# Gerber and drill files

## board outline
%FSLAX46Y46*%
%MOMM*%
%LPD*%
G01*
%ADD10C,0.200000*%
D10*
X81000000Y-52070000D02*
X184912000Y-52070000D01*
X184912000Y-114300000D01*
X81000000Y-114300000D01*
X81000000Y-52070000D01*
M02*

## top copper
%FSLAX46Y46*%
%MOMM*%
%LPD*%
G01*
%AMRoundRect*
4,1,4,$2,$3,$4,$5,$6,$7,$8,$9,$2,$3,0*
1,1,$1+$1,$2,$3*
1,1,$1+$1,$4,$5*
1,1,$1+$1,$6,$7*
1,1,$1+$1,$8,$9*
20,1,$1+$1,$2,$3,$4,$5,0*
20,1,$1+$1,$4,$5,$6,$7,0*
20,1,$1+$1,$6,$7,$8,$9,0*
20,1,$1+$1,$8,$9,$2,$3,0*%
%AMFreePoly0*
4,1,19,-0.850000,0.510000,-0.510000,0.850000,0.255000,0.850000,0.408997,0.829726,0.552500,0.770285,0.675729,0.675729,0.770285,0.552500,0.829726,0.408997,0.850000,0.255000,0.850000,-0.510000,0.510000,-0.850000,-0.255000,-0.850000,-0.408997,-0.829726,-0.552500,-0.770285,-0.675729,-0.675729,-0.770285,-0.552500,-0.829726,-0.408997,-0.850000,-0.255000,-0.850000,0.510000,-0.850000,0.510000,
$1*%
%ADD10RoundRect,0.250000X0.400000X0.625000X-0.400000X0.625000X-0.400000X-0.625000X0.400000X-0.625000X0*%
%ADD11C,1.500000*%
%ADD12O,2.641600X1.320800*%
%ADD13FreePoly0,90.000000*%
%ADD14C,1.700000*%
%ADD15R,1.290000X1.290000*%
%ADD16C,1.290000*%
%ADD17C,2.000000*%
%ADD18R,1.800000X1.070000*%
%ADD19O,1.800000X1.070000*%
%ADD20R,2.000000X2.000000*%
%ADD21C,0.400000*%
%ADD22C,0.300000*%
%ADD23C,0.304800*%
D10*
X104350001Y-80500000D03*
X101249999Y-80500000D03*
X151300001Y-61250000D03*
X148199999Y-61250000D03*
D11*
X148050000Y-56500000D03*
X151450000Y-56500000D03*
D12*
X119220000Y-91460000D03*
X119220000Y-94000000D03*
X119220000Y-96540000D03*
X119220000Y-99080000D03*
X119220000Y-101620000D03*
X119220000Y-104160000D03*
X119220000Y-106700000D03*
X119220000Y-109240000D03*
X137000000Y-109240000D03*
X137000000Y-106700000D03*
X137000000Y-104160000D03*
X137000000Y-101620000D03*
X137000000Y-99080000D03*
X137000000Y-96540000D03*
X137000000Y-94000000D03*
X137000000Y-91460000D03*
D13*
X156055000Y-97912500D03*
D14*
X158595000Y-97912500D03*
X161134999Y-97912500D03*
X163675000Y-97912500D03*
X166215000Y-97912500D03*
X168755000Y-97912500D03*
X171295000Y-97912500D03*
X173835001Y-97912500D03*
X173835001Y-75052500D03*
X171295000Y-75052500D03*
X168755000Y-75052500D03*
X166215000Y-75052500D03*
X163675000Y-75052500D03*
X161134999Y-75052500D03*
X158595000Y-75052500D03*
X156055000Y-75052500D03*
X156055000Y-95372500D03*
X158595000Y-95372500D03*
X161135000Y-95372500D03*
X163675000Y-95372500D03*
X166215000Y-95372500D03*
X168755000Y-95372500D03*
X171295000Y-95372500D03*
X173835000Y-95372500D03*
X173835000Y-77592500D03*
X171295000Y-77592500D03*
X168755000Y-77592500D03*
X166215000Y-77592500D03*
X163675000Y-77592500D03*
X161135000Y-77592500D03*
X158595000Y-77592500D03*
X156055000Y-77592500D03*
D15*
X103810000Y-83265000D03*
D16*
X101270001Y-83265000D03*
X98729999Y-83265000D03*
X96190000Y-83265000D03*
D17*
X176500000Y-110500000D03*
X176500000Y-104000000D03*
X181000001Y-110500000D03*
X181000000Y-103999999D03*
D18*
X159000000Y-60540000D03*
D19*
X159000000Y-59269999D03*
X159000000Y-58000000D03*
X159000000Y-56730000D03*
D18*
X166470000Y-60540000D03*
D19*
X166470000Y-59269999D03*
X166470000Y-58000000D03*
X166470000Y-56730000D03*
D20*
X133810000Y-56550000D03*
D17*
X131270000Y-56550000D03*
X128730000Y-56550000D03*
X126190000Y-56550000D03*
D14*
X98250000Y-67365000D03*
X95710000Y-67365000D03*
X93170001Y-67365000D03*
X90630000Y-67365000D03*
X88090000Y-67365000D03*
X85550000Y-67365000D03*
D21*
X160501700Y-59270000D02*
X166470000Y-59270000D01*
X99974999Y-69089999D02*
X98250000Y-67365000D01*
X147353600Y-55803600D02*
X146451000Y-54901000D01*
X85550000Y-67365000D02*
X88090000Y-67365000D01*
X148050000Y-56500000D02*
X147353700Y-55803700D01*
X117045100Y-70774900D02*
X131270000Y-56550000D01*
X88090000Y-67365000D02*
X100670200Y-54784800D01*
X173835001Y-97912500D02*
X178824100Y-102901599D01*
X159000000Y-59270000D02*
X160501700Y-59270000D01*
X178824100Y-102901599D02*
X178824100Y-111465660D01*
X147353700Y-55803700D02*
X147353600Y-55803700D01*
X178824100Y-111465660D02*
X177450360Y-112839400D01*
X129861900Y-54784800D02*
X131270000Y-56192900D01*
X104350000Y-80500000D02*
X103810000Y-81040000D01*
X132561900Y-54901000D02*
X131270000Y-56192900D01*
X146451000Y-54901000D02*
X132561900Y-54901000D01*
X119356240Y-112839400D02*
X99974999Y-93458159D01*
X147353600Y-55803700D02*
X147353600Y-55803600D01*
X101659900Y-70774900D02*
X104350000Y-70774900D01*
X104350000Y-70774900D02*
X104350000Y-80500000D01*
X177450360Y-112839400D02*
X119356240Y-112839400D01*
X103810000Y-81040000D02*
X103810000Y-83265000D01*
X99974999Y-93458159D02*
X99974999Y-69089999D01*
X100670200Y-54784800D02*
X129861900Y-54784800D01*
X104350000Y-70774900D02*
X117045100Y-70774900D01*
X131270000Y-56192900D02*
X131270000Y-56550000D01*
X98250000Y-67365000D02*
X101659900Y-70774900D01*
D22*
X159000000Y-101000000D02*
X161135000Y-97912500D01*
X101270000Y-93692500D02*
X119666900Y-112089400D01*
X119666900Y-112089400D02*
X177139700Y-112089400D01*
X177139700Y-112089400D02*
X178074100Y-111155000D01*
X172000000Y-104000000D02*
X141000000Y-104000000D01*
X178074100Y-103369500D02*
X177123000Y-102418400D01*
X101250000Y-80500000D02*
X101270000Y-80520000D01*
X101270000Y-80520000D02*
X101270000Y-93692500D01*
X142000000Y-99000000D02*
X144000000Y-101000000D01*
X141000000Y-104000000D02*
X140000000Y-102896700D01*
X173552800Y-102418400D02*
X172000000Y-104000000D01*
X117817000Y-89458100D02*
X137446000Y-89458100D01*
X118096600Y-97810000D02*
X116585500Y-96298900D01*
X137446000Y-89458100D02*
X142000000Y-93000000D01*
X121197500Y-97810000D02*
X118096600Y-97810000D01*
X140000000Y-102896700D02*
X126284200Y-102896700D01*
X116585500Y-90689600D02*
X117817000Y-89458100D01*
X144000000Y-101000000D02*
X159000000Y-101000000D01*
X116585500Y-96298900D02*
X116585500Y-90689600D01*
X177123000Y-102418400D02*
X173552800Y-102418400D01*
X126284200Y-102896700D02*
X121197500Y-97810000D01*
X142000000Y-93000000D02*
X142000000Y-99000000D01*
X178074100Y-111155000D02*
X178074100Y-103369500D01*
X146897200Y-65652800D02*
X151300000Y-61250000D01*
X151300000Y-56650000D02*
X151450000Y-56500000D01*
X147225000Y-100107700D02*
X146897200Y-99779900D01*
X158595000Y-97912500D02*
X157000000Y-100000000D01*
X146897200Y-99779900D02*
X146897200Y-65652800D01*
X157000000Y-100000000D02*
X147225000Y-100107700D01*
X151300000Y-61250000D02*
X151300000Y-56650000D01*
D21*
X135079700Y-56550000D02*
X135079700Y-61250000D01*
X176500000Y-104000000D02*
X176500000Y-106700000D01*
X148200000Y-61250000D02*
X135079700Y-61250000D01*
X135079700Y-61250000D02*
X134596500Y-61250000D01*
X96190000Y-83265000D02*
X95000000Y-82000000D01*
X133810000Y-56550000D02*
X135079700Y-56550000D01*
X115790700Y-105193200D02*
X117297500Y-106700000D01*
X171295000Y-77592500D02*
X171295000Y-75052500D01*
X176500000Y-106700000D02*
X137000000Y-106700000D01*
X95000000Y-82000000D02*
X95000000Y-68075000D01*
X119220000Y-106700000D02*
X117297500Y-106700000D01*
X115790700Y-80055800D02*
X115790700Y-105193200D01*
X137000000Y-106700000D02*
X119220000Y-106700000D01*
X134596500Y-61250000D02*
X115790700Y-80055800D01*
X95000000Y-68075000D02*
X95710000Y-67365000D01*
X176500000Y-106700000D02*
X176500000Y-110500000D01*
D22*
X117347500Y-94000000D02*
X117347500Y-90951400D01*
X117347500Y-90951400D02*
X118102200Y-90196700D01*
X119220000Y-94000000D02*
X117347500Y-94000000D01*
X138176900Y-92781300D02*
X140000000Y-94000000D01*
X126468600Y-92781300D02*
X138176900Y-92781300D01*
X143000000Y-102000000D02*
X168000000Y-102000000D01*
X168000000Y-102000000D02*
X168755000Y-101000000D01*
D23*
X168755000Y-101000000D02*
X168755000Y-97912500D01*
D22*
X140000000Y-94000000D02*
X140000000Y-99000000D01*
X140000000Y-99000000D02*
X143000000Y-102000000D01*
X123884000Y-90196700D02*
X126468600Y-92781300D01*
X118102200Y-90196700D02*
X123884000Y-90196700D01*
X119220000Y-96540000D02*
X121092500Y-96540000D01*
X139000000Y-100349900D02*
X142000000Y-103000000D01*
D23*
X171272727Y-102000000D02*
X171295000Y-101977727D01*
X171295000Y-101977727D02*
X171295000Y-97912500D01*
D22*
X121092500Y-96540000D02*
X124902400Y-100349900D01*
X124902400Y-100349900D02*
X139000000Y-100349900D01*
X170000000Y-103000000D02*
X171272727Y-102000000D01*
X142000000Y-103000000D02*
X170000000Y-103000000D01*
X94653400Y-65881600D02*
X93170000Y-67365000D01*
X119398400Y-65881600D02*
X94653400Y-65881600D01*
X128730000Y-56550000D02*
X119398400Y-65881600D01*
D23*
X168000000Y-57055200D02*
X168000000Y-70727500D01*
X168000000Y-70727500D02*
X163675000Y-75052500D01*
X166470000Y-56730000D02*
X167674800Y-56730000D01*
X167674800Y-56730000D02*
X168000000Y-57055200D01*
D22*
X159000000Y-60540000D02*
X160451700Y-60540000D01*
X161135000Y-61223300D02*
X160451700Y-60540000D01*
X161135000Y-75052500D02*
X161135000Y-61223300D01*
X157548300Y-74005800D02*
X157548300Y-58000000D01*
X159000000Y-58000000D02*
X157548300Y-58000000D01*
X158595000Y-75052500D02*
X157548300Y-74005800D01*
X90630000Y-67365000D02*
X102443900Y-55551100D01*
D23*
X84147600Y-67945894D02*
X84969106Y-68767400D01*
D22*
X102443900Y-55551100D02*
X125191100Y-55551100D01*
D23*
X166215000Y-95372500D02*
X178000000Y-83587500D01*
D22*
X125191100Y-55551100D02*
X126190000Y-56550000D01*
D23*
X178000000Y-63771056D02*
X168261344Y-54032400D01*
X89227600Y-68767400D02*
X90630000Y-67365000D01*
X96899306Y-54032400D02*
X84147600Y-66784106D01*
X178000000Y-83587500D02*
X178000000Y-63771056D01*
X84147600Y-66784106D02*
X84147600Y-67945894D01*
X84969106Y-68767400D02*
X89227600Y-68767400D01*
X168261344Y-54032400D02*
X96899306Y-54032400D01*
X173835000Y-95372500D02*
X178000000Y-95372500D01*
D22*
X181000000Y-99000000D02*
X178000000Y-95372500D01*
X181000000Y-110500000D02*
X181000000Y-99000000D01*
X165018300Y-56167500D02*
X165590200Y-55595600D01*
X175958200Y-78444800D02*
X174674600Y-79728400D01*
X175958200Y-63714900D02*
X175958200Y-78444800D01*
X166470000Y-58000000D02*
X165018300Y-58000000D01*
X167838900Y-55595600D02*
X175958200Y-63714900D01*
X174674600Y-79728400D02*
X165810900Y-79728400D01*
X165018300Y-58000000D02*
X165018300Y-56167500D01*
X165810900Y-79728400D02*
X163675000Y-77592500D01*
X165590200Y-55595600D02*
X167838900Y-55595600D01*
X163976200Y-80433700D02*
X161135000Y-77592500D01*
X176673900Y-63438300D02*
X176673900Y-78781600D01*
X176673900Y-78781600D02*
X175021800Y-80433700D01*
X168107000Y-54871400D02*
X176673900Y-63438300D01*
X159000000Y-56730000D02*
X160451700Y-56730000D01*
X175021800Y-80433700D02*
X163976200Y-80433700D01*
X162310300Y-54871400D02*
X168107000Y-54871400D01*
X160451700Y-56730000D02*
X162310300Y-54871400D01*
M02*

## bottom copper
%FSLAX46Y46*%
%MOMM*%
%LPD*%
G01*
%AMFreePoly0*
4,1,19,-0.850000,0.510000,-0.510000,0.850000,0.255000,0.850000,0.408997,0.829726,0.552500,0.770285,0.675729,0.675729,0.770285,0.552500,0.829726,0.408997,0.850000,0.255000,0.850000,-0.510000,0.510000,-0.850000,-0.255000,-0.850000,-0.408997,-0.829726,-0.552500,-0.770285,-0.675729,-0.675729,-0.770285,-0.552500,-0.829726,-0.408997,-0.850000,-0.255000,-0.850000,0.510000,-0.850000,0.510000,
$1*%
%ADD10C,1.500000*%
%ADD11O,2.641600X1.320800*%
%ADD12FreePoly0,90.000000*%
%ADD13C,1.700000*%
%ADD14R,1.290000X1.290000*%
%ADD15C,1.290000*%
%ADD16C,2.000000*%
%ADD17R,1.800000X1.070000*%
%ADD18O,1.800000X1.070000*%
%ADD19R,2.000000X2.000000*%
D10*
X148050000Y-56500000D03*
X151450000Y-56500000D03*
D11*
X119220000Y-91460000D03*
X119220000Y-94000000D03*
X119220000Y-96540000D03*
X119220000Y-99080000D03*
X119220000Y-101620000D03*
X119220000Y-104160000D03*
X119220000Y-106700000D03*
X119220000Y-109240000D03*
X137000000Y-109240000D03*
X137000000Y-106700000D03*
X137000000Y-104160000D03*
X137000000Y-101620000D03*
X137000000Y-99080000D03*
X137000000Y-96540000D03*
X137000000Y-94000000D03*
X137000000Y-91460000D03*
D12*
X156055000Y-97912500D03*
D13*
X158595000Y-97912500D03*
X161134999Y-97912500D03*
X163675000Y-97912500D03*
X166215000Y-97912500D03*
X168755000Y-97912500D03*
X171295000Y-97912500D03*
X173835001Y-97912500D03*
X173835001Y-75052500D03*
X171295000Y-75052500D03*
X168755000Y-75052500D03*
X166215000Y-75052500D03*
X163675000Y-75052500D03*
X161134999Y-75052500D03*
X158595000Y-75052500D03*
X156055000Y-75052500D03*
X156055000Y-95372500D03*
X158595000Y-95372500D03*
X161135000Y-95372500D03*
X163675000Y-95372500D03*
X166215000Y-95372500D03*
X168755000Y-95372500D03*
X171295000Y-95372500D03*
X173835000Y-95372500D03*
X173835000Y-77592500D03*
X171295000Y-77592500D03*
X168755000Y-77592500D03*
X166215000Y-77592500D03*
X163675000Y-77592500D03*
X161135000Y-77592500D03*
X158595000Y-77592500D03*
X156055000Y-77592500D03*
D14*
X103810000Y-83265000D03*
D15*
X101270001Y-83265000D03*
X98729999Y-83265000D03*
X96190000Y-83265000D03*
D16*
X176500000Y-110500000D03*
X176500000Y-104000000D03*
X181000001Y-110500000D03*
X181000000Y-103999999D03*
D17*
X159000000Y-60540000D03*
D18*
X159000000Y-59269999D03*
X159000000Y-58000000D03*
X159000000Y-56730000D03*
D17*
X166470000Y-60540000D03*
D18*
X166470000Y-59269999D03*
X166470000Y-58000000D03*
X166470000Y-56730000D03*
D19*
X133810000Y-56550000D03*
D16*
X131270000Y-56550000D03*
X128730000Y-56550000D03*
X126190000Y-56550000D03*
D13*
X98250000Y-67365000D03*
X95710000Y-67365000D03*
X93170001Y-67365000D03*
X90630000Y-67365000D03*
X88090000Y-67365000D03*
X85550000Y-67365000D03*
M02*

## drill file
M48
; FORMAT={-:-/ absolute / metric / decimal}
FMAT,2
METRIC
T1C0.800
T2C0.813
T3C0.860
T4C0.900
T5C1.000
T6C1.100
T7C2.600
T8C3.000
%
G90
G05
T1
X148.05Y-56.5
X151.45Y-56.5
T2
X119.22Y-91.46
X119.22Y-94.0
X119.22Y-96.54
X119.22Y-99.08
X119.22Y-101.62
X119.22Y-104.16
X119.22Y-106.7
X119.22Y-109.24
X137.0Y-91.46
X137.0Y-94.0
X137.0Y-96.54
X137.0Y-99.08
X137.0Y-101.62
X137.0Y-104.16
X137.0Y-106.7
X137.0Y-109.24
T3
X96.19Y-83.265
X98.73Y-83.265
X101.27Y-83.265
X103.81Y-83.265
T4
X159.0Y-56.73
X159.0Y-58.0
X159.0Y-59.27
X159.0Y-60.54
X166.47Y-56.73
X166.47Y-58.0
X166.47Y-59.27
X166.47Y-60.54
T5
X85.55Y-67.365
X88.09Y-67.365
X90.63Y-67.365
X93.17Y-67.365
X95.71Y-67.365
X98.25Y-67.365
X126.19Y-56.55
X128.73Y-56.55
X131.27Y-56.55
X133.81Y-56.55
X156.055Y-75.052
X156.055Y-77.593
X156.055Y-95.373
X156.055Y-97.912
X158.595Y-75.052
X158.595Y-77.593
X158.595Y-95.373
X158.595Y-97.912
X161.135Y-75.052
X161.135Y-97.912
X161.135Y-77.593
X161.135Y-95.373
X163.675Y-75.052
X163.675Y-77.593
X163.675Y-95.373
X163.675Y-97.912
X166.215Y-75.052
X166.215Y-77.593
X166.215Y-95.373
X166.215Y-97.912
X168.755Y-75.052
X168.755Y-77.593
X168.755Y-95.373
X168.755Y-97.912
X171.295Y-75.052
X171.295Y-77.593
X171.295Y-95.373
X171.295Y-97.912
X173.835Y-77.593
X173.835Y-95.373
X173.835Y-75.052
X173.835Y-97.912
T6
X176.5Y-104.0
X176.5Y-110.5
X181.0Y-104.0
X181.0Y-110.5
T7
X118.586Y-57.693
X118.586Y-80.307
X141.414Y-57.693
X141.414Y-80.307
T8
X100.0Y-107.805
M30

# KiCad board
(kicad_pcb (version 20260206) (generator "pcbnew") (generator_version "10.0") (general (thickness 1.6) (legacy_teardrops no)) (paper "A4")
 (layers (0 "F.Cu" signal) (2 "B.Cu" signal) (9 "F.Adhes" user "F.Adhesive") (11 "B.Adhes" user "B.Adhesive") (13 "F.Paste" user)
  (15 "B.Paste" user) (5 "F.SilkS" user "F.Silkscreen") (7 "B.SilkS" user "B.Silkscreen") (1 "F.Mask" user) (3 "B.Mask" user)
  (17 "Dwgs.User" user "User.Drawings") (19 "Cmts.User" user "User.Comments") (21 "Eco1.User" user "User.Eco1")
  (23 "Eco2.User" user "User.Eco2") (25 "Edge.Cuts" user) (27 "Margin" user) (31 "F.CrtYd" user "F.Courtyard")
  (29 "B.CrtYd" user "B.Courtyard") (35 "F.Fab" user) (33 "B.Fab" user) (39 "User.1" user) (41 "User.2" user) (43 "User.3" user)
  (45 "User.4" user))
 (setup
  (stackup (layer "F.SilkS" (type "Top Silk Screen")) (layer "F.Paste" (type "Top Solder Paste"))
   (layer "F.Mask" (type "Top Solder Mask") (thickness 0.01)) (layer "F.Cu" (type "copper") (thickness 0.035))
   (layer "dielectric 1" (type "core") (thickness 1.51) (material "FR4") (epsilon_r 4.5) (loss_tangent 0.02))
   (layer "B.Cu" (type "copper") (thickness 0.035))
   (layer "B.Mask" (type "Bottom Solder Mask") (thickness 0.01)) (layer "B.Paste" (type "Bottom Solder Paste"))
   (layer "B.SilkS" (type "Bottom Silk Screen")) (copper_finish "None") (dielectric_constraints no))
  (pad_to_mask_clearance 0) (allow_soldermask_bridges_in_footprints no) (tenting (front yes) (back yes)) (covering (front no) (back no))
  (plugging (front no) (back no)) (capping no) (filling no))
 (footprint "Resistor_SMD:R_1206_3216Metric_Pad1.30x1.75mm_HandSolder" (layer "F.Cu") (at 102.8 80.5 180)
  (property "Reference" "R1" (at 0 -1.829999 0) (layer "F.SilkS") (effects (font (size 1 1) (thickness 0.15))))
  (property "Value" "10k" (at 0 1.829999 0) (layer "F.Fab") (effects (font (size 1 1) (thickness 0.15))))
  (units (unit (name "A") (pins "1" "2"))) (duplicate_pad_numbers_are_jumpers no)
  (pad "1" smd roundrect (at -1.550001 0 180) (size 1.3 1.75) (layers "F.Cu" "F.Mask" "F.Paste") (roundrect_rratio 0.192308) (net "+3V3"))
  (pad "2" smd roundrect (at 1.550001 0 180) (size 1.3 1.75) (layers "F.Cu" "F.Mask" "F.Paste") (roundrect_rratio 0.192308)
   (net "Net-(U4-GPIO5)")))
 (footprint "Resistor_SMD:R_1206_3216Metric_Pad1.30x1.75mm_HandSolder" (layer "F.Cu") (at 149.75 61.25 180)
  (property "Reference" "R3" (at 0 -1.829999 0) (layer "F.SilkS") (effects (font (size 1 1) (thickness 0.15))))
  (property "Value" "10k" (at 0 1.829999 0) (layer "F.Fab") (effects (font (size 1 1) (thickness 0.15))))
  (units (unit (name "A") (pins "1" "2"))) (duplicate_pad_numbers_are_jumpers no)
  (pad "1" smd roundrect (at -1.550001 0 180) (size 1.3 1.75) (layers "F.Cu" "F.Mask" "F.Paste") (roundrect_rratio 0.192308)
   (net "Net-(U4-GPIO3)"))
  (pad "2" smd roundrect (at 1.550001 0 180) (size 1.3 1.75) (layers "F.Cu" "F.Mask" "F.Paste") (roundrect_rratio 0.192308) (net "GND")))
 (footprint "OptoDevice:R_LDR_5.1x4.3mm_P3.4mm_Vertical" (layer "F.Cu") (at 148.05 56.5)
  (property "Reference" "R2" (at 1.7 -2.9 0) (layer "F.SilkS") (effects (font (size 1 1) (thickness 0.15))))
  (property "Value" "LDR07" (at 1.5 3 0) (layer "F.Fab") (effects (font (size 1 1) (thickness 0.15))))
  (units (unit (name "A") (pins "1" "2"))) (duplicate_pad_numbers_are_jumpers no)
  (pad "1" thru_hole circle (at 0 0) (size 1.5 1.5) (drill 0.8) (layers "*.Cu" "*.Mask") (remove_unused_layers no) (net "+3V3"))
  (pad "2" thru_hole circle (at 3.4 0) (size 1.5 1.5) (drill 0.8) (layers "*.Cu" "*.Mask") (remove_unused_layers no) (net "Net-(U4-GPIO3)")))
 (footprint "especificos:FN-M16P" (layer "F.Cu") (at 128.11 100.35 -90)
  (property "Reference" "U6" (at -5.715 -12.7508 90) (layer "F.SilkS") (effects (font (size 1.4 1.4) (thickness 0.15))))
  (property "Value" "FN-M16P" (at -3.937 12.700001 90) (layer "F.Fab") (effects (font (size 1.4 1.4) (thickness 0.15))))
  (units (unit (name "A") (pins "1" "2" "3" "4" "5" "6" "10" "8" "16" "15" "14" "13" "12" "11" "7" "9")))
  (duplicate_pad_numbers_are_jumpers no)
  (pad "1" thru_hole oval (at -8.89 8.89 270) (size 1.3208 2.6416) (drill 0.8128) (layers "*.Cu" "*.Mask") (remove_unused_layers no)
   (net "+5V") (solder_mask_margin 0.102))
  (pad "2" thru_hole oval (at -6.35 8.89 270) (size 1.3208 2.6416) (drill 0.8128) (layers "*.Cu" "*.Mask") (remove_unused_layers no)
   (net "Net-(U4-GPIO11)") (solder_mask_margin 0.102))
  (pad "3" thru_hole oval (at -3.81 8.89 270) (size 1.3208 2.6416) (drill 0.8128) (layers "*.Cu" "*.Mask") (remove_unused_layers no)
   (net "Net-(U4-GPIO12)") (solder_mask_margin 0.102))
  (pad "4" thru_hole oval (at -1.27 8.89 270) (size 1.3208 2.6416) (drill 0.8128) (layers "*.Cu" "*.Mask") (remove_unused_layers no)
   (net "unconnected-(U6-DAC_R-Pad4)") (solder_mask_margin 0.102))
  (pad "5" thru_hole oval (at 1.27 8.89 270) (size 1.3208 2.6416) (drill 0.8128) (layers "*.Cu" "*.Mask") (remove_unused_layers no)
   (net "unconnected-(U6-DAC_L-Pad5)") (solder_mask_margin 0.102))
  (pad "6" thru_hole oval (at 3.81 8.89 270) (size 1.3208 2.6416) (drill 0.8128) (layers "*.Cu" "*.Mask") (remove_unused_layers no)
   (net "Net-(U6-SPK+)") (solder_mask_margin 0.102))
  (pad "7" thru_hole oval (at 6.35 8.89 270) (size 1.3208 2.6416) (drill 0.8128) (layers "*.Cu" "*.Mask") (remove_unused_layers no)
   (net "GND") (solder_mask_margin 0.102))
  (pad "8" thru_hole oval (at 8.89 8.89 270) (size 1.3208 2.6416) (drill 0.8128) (layers "*.Cu" "*.Mask") (remove_unused_layers no)
   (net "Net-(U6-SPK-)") (solder_mask_margin 0.102))
  (pad "9" thru_hole oval (at 8.89 -8.89 270) (size 1.3208 2.6416) (drill 0.8128) (layers "*.Cu" "*.Mask") (remove_unused_layers no)
   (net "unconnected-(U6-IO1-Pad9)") (solder_mask_margin 0.102))
  (pad "10" thru_hole oval (at 6.35 -8.89 270) (size 1.3208 2.6416) (drill 0.8128) (layers "*.Cu" "*.Mask") (remove_unused_layers no)
   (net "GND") (solder_mask_margin 0.102))
  (pad "11" thru_hole oval (at 3.81 -8.89 270) (size 1.3208 2.6416) (drill 0.8128) (layers "*.Cu" "*.Mask") (remove_unused_layers no)
   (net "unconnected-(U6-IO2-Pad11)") (solder_mask_margin 0.102))
  (pad "12" thru_hole oval (at 1.27 -8.89 270) (size 1.3208 2.6416) (drill 0.8128) (layers "*.Cu" "*.Mask") (remove_unused_layers no)
   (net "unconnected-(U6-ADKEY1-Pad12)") (solder_mask_margin 0.102))
  (pad "13" thru_hole oval (at -1.27 -8.89 270) (size 1.3208 2.6416) (drill 0.8128) (layers "*.Cu" "*.Mask") (remove_unused_layers no)
   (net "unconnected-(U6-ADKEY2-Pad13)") (solder_mask_margin 0.102))
  (pad "14" thru_hole oval (at -3.81 -8.89 270) (size 1.3208 2.6416) (drill 0.8128) (layers "*.Cu" "*.Mask") (remove_unused_layers no)
   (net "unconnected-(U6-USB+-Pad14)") (solder_mask_margin 0.102))
  (pad "15" thru_hole oval (at -6.35 -8.89 270) (size 1.3208 2.6416) (drill 0.8128) (layers "*.Cu" "*.Mask") (remove_unused_layers no)
   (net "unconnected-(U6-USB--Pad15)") (solder_mask_margin 0.102))
  (pad "16" thru_hole oval (at -8.89 -8.89 270) (size 1.3208 2.6416) (drill 0.8128) (layers "*.Cu" "*.Mask") (remove_unused_layers no)
   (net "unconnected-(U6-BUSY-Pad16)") (solder_mask_margin 0.102)))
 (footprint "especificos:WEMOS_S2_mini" (layer "F.Cu") (at 156.055 97.9125 90)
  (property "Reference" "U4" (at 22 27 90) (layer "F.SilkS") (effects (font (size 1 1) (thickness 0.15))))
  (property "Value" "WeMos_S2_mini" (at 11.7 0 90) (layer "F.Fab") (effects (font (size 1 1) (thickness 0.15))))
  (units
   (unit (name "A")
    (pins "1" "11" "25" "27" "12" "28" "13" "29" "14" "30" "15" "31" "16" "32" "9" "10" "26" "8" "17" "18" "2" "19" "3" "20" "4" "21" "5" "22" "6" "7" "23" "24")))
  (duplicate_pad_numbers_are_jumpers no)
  (pad "1" thru_hole roundrect (at 0 0 90) (size 1.7 1.7) (drill 1) (layers "*.Cu" "*.Mask") (remove_unused_layers no)
   (roundrect_rratio 0.35) (chamfer_ratio 0.2) (chamfer top_left bottom_right) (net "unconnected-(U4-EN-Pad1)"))
  (pad "2" thru_hole circle (at 0 2.54 90) (size 1.7 1.7) (drill 1) (layers "*.Cu" "*.Mask") (remove_unused_layers no)
   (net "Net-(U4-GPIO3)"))
  (pad "3" thru_hole circle (at 0 5.079999 90) (size 1.7 1.7) (drill 1) (layers "*.Cu" "*.Mask") (remove_unused_layers no)
   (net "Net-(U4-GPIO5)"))
  (pad "4" thru_hole circle (at 0 7.62 90) (size 1.7 1.7) (drill 1) (layers "*.Cu" "*.Mask") (remove_unused_layers no)
   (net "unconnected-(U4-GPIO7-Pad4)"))
  (pad "5" thru_hole circle (at 0 10.16 90) (size 1.7 1.7) (drill 1) (layers "*.Cu" "*.Mask") (remove_unused_layers no) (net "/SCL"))
  (pad "6" thru_hole circle (at 0 12.7 90) (size 1.7 1.7) (drill 1) (layers "*.Cu" "*.Mask") (remove_unused_layers no)
   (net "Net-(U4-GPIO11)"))
  (pad "7" thru_hole circle (at 0 15.24 90) (size 1.7 1.7) (drill 1) (layers "*.Cu" "*.Mask") (remove_unused_layers no)
   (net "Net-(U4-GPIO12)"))
  (pad "8" thru_hole circle (at 0 17.780001 90) (size 1.7 1.7) (drill 1) (layers "*.Cu" "*.Mask") (remove_unused_layers no) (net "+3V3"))
  (pad "9" thru_hole circle (at 22.86 17.780001 90) (size 1.7 1.7) (drill 1) (layers "*.Cu" "*.Mask") (remove_unused_layers no) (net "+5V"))
  (pad "10" thru_hole circle (at 22.86 15.24 90) (size 1.7 1.7) (drill 1) (layers "*.Cu" "*.Mask") (remove_unused_layers no) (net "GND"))
  (pad "11" thru_hole circle (at 22.86 12.7 90) (size 1.7 1.7) (drill 1) (layers "*.Cu" "*.Mask") (remove_unused_layers no)
   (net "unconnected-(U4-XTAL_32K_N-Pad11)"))
  (pad "12" thru_hole circle (at 22.86 10.16 90) (size 1.7 1.7) (drill 1) (layers "*.Cu" "*.Mask") (remove_unused_layers no)
   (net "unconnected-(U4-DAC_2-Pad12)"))
  (pad "13" thru_hole circle (at 22.86 7.62 90) (size 1.7 1.7) (drill 1) (layers "*.Cu" "*.Mask") (remove_unused_layers no)
   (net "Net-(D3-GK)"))
  (pad "14" thru_hole circle (at 22.86 5.079999 90) (size 1.7 1.7) (drill 1) (layers "*.Cu" "*.Mask") (remove_unused_layers no)
   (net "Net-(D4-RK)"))
  (pad "15" thru_hole circle (at 22.86 2.54 90) (size 1.7 1.7) (drill 1) (layers "*.Cu" "*.Mask") (remove_unused_layers no)
   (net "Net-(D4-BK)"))
  (pad "16" thru_hole circle (at 22.86 0 90) (size 1.7 1.7) (drill 1) (layers "*.Cu" "*.Mask") (remove_unused_layers no)
   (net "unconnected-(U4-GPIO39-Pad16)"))
  (pad "17" thru_hole circle (at 2.54 0 90) (size 1.7 1.7) (drill 1) (layers "*.Cu" "*.Mask") (remove_unused_layers no)
   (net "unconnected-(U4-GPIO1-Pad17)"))
  (pad "18" thru_hole circle (at 2.54 2.54 90) (size 1.7 1.7) (drill 1) (layers "*.Cu" "*.Mask") (remove_unused_layers no)
   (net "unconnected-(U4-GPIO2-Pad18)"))
  (pad "19" thru_hole circle (at 2.54 5.08 90) (size 1.7 1.7) (drill 1) (layers "*.Cu" "*.Mask") (remove_unused_layers no)
   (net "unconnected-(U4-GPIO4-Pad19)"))
  (pad "20" thru_hole circle (at 2.54 7.62 90) (size 1.7 1.7) (drill 1) (layers "*.Cu" "*.Mask") (remove_unused_layers no)
   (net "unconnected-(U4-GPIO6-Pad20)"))
  (pad "21" thru_hole circle (at 2.54 10.16 90) (size 1.7 1.7) (drill 1) (layers "*.Cu" "*.Mask") (remove_unused_layers no) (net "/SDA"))
  (pad "22" thru_hole circle (at 2.54 12.7 90) (size 1.7 1.7) (drill 1) (layers "*.Cu" "*.Mask") (remove_unused_layers no)
   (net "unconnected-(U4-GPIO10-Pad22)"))
  (pad "23" thru_hole circle (at 2.54 15.24 90) (size 1.7 1.7) (drill 1) (layers "*.Cu" "*.Mask") (remove_unused_layers no)
   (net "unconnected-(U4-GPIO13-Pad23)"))
  (pad "24" thru_hole circle (at 2.54 17.78 90) (size 1.7 1.7) (drill 1) (layers "*.Cu" "*.Mask") (remove_unused_layers no)
   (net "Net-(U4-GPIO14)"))
  (pad "25" thru_hole circle (at 20.32 17.78 90) (size 1.7 1.7) (drill 1) (layers "*.Cu" "*.Mask") (remove_unused_layers no)
   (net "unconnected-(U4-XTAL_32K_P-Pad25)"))
  (pad "26" thru_hole circle (at 20.32 15.24 90) (size 1.7 1.7) (drill 1) (layers "*.Cu" "*.Mask") (remove_unused_layers no) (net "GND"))
  (pad "27" thru_hole circle (at 20.32 12.7 90) (size 1.7 1.7) (drill 1) (layers "*.Cu" "*.Mask") (remove_unused_layers no)
   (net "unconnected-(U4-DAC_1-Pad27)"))
  (pad "28" thru_hole circle (at 20.32 10.16 90) (size 1.7 1.7) (drill 1) (layers "*.Cu" "*.Mask") (remove_unused_layers no)
   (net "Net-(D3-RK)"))
  (pad "29" thru_hole circle (at 20.32 7.62 90) (size 1.7 1.7) (drill 1) (layers "*.Cu" "*.Mask") (remove_unused_layers no)
   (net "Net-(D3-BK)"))
  (pad "30" thru_hole circle (at 20.32 5.08 90) (size 1.7 1.7) (drill 1) (layers "*.Cu" "*.Mask") (remove_unused_layers no)
   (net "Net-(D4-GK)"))
  (pad "31" thru_hole circle (at 20.32 2.54 90) (size 1.7 1.7) (drill 1) (layers "*.Cu" "*.Mask") (remove_unused_layers no)
   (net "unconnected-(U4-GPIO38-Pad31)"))
  (pad "32" thru_hole circle (at 20.32 0 90) (size 1.7 1.7) (drill 1) (layers "*.Cu" "*.Mask") (remove_unused_layers no)
   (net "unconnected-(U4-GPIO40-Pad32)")))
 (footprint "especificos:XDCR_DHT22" (layer "F.Cu") (at 100 98.455 180)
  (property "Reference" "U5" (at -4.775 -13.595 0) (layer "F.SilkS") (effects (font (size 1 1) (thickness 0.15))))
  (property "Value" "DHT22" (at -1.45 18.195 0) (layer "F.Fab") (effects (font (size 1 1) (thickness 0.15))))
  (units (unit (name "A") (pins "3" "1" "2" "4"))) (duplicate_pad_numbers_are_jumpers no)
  (pad "" np_thru_hole circle (at 0 -9.349999 180) (size 3 3) (drill 3) (layers "*.Cu" "*.Mask"))
  (pad "1" thru_hole rect (at -3.81 15.19 180) (size 1.29 1.29) (drill 0.86) (layers "*.Cu" "*.Mask") (remove_unused_layers no) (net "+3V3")
   (solder_mask_margin 0.102))
  (pad "2" thru_hole circle (at -1.270001 15.19 180) (size 1.29 1.29) (drill 0.86) (layers "*.Cu" "*.Mask") (remove_unused_layers no)
   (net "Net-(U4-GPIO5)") (solder_mask_margin 0.102))
  (pad "3" thru_hole circle (at 1.270001 15.19 180) (size 1.29 1.29) (drill 0.86) (layers "*.Cu" "*.Mask") (remove_unused_layers no)
   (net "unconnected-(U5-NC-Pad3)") (solder_mask_margin 0.102))
  (pad "4" thru_hole circle (at 3.81 15.19 180) (size 1.29 1.29) (drill 0.86) (layers "*.Cu" "*.Mask") (remove_unused_layers no) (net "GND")
   (solder_mask_margin 0.102)))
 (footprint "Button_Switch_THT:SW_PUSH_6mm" (layer "F.Cu") (at 176.5 110.5 90)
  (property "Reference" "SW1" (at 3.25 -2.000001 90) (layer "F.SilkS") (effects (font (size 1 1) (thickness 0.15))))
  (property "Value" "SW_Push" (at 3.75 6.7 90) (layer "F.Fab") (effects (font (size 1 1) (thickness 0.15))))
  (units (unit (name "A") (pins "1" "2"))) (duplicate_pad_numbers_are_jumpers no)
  (pad "1" thru_hole circle (at 0 0 180) (size 2 2) (drill 1.1) (layers "*.Cu" "*.Mask") (remove_unused_layers no) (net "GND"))
  (pad "1" thru_hole circle (at 6.5 0 180) (size 2 2) (drill 1.1) (layers "*.Cu" "*.Mask") (remove_unused_layers no) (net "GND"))
  (pad "2" thru_hole circle (at 0 4.500001 180) (size 2 2) (drill 1.1) (layers "*.Cu" "*.Mask") (remove_unused_layers no)
   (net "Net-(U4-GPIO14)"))
  (pad "2" thru_hole circle (at 6.500001 4.5 180) (size 2 2) (drill 1.1) (layers "*.Cu" "*.Mask") (remove_unused_layers no)
   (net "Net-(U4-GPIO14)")))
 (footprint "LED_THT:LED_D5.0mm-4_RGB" (layer "B.Cu") (at 159 60.54 90)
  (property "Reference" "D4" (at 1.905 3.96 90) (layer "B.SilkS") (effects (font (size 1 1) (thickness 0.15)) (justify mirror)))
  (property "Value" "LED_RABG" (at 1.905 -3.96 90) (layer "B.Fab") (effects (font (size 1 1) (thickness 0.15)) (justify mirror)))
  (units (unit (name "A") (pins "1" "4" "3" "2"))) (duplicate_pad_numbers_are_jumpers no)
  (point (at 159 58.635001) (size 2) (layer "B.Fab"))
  (pad "1" thru_hole rect (at 0 0 90) (size 1.07 1.8) (drill 0.9) (layers "*.Cu" "*.Mask") (remove_unused_layers no) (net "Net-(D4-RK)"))
  (pad "2" thru_hole oval (at 1.270001 0 90) (size 1.07 1.8) (drill 0.9) (layers "*.Cu" "*.Mask") (remove_unused_layers no) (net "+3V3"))
  (pad "3" thru_hole oval (at 2.54 0 90) (size 1.07 1.8) (drill 0.9) (layers "*.Cu" "*.Mask") (remove_unused_layers no) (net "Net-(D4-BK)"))
  (pad "4" thru_hole oval (at 3.81 0 90) (size 1.07 1.8) (drill 0.9) (layers "*.Cu" "*.Mask") (remove_unused_layers no) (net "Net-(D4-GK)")))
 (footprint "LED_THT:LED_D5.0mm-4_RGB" (layer "B.Cu") (at 166.47 60.54 90)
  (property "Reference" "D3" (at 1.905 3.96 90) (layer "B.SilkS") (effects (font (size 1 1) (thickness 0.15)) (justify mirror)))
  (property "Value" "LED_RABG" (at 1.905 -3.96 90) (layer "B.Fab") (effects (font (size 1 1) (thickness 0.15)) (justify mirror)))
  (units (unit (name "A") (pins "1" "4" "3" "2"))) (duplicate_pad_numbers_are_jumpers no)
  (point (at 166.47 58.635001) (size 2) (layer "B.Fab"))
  (pad "1" thru_hole rect (at 0 0 90) (size 1.07 1.8) (drill 0.9) (layers "*.Cu" "*.Mask") (remove_unused_layers no) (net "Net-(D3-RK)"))
  (pad "2" thru_hole oval (at 1.270001 0 90) (size 1.07 1.8) (drill 0.9) (layers "*.Cu" "*.Mask") (remove_unused_layers no) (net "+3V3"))
  (pad "3" thru_hole oval (at 2.54 0 90) (size 1.07 1.8) (drill 0.9) (layers "*.Cu" "*.Mask") (remove_unused_layers no) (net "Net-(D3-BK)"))
  (pad "4" thru_hole oval (at 3.81 0 90) (size 1.07 1.8) (drill 0.9) (layers "*.Cu" "*.Mask") (remove_unused_layers no) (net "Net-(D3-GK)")))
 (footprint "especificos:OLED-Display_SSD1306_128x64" (layer "B.Cu") (at 130 69.25 180)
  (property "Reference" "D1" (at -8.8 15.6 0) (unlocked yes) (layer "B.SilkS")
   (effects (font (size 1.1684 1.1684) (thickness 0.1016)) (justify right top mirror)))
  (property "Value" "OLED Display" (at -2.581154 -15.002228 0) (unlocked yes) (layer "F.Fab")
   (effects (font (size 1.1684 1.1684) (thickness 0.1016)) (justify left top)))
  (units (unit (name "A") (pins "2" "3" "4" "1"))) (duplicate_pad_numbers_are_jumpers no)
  (pad "" np_thru_hole circle (at -11.414 -11.057 180) (size 2.6 2.6) (drill 2.6) (layers "*.Cu" "*.Mask"))
  (pad "" np_thru_hole circle (at -11.414 11.557 180) (size 2.6 2.6) (drill 2.6) (layers "*.Cu" "*.Mask"))
  (pad "" np_thru_hole circle (at 11.414 -11.057 180) (size 2.6 2.6) (drill 2.6) (layers "*.Cu" "*.Mask"))
  (pad "" np_thru_hole circle (at 11.414 11.557 180) (size 2.6 2.6) (drill 2.6) (layers "*.Cu" "*.Mask"))
  (pad "1" thru_hole rect (at -3.81 12.7 180) (size 2 2) (drill 1) (layers "*.Cu" "*.Mask") (remove_unused_layers no) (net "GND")
   (thermal_bridge_angle 0))
  (pad "2" thru_hole circle (at -1.27 12.7 180) (size 2 2) (drill 1) (layers "*.Cu" "*.Mask") (remove_unused_layers no) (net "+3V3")
   (thermal_bridge_angle 0))
  (pad "3" thru_hole circle (at 1.27 12.7 180) (size 2 2) (drill 1) (layers "*.Cu" "*.Mask") (remove_unused_layers no) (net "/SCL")
   (thermal_bridge_angle 0))
  (pad "4" thru_hole circle (at 3.81 12.7 180) (size 2 2) (drill 1) (layers "*.Cu" "*.Mask") (remove_unused_layers no) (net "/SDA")
   (thermal_bridge_angle 0)))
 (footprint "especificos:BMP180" (layer "B.Cu") (at 98.25 67.365 90)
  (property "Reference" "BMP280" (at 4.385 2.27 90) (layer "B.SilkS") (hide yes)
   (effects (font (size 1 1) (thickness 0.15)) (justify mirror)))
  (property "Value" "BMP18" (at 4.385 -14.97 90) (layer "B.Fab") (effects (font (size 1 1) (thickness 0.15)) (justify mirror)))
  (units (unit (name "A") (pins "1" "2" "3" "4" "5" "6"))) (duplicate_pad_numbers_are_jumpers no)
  (pad "1" thru_hole circle (at 0 0 90) (size 1.7 1.7) (drill 1) (layers "*.Cu" "*.Mask") (remove_unused_layers no) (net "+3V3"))
  (pad "2" thru_hole circle (at 0 -2.54 90) (size 1.7 1.7) (drill 1) (layers "*.Cu" "*.Mask") (remove_unused_layers no) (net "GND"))
  (pad "3" thru_hole circle (at 0 -5.079999 90) (size 1.7 1.7) (drill 1) (layers "*.Cu" "*.Mask") (remove_unused_layers no) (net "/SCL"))
  (pad "4" thru_hole circle (at 0 -7.62 90) (size 1.7 1.7) (drill 1) (layers "*.Cu" "*.Mask") (remove_unused_layers no) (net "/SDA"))
  (pad "5" thru_hole circle (at 0 -10.16 90) (size 1.7 1.7) (drill 1) (layers "*.Cu" "*.Mask") (remove_unused_layers no) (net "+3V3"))
  (pad "6" thru_hole circle (at 0 -12.7 90) (size 1.7 1.7) (drill 1) (layers "*.Cu" "*.Mask") (remove_unused_layers no) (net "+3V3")))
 (gr_rect (start 81 52.07) (end 184.912 114.3) (stroke (width 0.2) (type default)) (fill no) (layer "Edge.Cuts"))
 (segment (start 160.5017 59.27) (end 166.47 59.27) (width 0.4) (layer "F.Cu") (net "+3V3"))
 (segment (start 99.974999 69.089999) (end 98.25 67.365) (width 0.4) (layer "F.Cu") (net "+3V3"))
 (segment (start 147.3536 55.8036) (end 146.451 54.901) (width 0.4) (layer "F.Cu") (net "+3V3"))
 (segment (start 85.55 67.365) (end 88.09 67.365) (width 0.4) (layer "F.Cu") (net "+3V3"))
 (segment (start 148.05 56.5) (end 147.3537 55.8037) (width 0.4) (layer "F.Cu") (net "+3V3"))
 (segment (start 117.0451 70.7749) (end 131.27 56.55) (width 0.4) (layer "F.Cu") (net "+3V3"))
 (segment (start 88.09 67.365) (end 100.6702 54.7848) (width 0.4) (layer "F.Cu") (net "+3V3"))
 (segment (start 173.835001 97.9125) (end 178.8241 102.901599) (width 0.4) (layer "F.Cu") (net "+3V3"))
 (segment (start 159 59.27) (end 160.5017 59.27) (width 0.4) (layer "F.Cu") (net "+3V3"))
 (segment (start 178.8241 102.901599) (end 178.8241 111.46566) (width 0.4) (layer "F.Cu") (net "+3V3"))
 (segment (start 147.3537 55.8037) (end 147.3536 55.8037) (width 0.4) (layer "F.Cu") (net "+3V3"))
 (segment (start 178.8241 111.46566) (end 177.45036 112.8394) (width 0.4) (layer "F.Cu") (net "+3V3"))
 (segment (start 129.8619 54.7848) (end 131.27 56.1929) (width 0.4) (layer "F.Cu") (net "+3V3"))
 (segment (start 104.35 80.5) (end 103.81 81.04) (width 0.4) (layer "F.Cu") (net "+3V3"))
 (segment (start 132.5619 54.901) (end 131.27 56.1929) (width 0.4) (layer "F.Cu") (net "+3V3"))
 (segment (start 146.451 54.901) (end 132.5619 54.901) (width 0.4) (layer "F.Cu") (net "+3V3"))
 (segment (start 119.35624 112.8394) (end 99.974999 93.458159) (width 0.4) (layer "F.Cu") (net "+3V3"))
 (segment (start 147.3536 55.8037) (end 147.3536 55.8036) (width 0.4) (layer "F.Cu") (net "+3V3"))
 (segment (start 101.6599 70.7749) (end 104.35 70.7749) (width 0.4) (layer "F.Cu") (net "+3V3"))
 (segment (start 104.35 70.7749) (end 104.35 80.5) (width 0.4) (layer "F.Cu") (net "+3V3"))
 (segment (start 177.45036 112.8394) (end 119.35624 112.8394) (width 0.4) (layer "F.Cu") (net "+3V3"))
 (segment (start 103.81 81.04) (end 103.81 83.265) (width 0.4) (layer "F.Cu") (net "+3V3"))
 (segment (start 99.974999 93.458159) (end 99.974999 69.089999) (width 0.4) (layer "F.Cu") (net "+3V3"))
 (segment (start 100.6702 54.7848) (end 129.8619 54.7848) (width 0.4) (layer "F.Cu") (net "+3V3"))
 (segment (start 104.35 70.7749) (end 117.0451 70.7749) (width 0.4) (layer "F.Cu") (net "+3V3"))
 (segment (start 131.27 56.1929) (end 131.27 56.55) (width 0.4) (layer "F.Cu") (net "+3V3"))
 (segment (start 98.25 67.365) (end 101.6599 70.7749) (width 0.4) (layer "F.Cu") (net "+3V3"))
 (segment (start 159 101) (end 161.135 97.9125) (width 0.3) (layer "F.Cu") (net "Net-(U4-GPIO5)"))
 (segment (start 101.27 93.6925) (end 119.6669 112.0894) (width 0.3) (layer "F.Cu") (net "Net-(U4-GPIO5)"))
 (segment (start 119.6669 112.0894) (end 177.1397 112.0894) (width 0.3) (layer "F.Cu") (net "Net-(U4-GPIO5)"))
 (segment (start 177.1397 112.0894) (end 178.0741 111.155) (width 0.3) (layer "F.Cu") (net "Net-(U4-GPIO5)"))
 (segment (start 172 104) (end 141 104) (width 0.3) (layer "F.Cu") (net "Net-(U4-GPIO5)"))
 (segment (start 178.0741 103.3695) (end 177.123 102.4184) (width 0.3) (layer "F.Cu") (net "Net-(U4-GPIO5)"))
 (segment (start 101.25 80.5) (end 101.27 80.52) (width 0.3) (layer "F.Cu") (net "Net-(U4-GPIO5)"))
 (segment (start 101.27 80.52) (end 101.27 93.6925) (width 0.3) (layer "F.Cu") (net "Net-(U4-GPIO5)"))
 (segment (start 142 99) (end 144 101) (width 0.3) (layer "F.Cu") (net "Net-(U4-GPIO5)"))
 (segment (start 141 104) (end 140 102.8967) (width 0.3) (layer "F.Cu") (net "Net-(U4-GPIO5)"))
 (segment (start 173.5528 102.4184) (end 172 104) (width 0.3) (layer "F.Cu") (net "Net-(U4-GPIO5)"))
 (segment (start 117.817 89.4581) (end 137.446 89.4581) (width 0.3) (layer "F.Cu") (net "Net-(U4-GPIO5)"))
 (segment (start 118.0966 97.81) (end 116.5855 96.2989) (width 0.3) (layer "F.Cu") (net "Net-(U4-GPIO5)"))
 (segment (start 137.446 89.4581) (end 142 93) (width 0.3) (layer "F.Cu") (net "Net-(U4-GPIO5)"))
 (segment (start 121.1975 97.81) (end 118.0966 97.81) (width 0.3) (layer "F.Cu") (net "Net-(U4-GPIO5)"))
 (segment (start 140 102.8967) (end 126.2842 102.8967) (width 0.3) (layer "F.Cu") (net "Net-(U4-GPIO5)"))
 (segment (start 116.5855 90.6896) (end 117.817 89.4581) (width 0.3) (layer "F.Cu") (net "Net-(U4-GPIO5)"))
 (segment (start 144 101) (end 159 101) (width 0.3) (layer "F.Cu") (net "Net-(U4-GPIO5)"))
 (segment (start 116.5855 96.2989) (end 116.5855 90.6896) (width 0.3) (layer "F.Cu") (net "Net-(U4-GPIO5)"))
 (segment (start 177.123 102.4184) (end 173.5528 102.4184) (width 0.3) (layer "F.Cu") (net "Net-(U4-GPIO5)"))
 (segment (start 126.2842 102.8967) (end 121.1975 97.81) (width 0.3) (layer "F.Cu") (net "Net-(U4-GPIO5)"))
 (segment (start 142 93) (end 142 99) (width 0.3) (layer "F.Cu") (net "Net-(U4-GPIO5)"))
 (segment (start 178.0741 111.155) (end 178.0741 103.3695) (width 0.3) (layer "F.Cu") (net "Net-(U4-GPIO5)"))
 (segment (start 146.8972 65.6528) (end 151.3 61.25) (width 0.3) (layer "F.Cu") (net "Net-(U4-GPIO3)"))
 (segment (start 151.3 56.65) (end 151.45 56.5) (width 0.3) (layer "F.Cu") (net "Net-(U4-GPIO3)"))
 (segment (start 147.225 100.1077) (end 146.8972 99.7799) (width 0.3) (layer "F.Cu") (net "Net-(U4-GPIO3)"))
 (segment (start 158.595 97.9125) (end 157 100) (width 0.3) (layer "F.Cu") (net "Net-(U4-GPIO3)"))
 (segment (start 146.8972 99.7799) (end 146.8972 65.6528) (width 0.3) (layer "F.Cu") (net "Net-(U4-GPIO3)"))
 (segment (start 157 100) (end 147.225 100.1077) (width 0.3) (layer "F.Cu") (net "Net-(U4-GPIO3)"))
 (segment (start 151.3 61.25) (end 151.3 56.65) (width 0.3) (layer "F.Cu") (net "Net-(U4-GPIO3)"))
 (segment (start 135.0797 56.55) (end 135.0797 61.25) (width 0.4) (layer "F.Cu") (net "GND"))
 (segment (start 176.5 104) (end 176.5 106.7) (width 0.4) (layer "F.Cu") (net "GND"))
 (segment (start 148.2 61.25) (end 135.0797 61.25) (width 0.4) (layer "F.Cu") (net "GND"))
 (segment (start 135.0797 61.25) (end 134.5965 61.25) (width 0.4) (layer "F.Cu") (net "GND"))
 (segment (start 96.19 83.265) (end 95 82) (width 0.4) (layer "F.Cu") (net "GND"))
 (segment (start 133.81 56.55) (end 135.0797 56.55) (width 0.4) (layer "F.Cu") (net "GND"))
 (segment (start 115.7907 105.1932) (end 117.2975 106.7) (width 0.4) (layer "F.Cu") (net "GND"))
 (segment (start 171.295 77.5925) (end 171.295 75.0525) (width 0.4) (layer "F.Cu") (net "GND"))
 (segment (start 176.5 106.7) (end 137 106.7) (width 0.4) (layer "F.Cu") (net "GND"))
 (segment (start 95 82) (end 95 68.075) (width 0.4) (layer "F.Cu") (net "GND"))
 (segment (start 119.22 106.7) (end 117.2975 106.7) (width 0.4) (layer "F.Cu") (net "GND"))
 (segment (start 115.7907 80.0558) (end 115.7907 105.1932) (width 0.4) (layer "F.Cu") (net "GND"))
 (segment (start 137 106.7) (end 119.22 106.7) (width 0.4) (layer "F.Cu") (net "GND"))
 (segment (start 134.5965 61.25) (end 115.7907 80.0558) (width 0.4) (layer "F.Cu") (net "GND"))
 (segment (start 95 68.075) (end 95.71 67.365) (width 0.4) (layer "F.Cu") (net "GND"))
 (segment (start 176.5 106.7) (end 176.5 110.5) (width 0.4) (layer "F.Cu") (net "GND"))
 (segment (start 117.3475 94) (end 117.3475 90.9514) (width 0.3) (layer "F.Cu") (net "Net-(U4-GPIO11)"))
 (segment (start 117.3475 90.9514) (end 118.1022 90.1967) (width 0.3) (layer "F.Cu") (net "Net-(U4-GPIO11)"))
 (segment (start 119.22 94) (end 117.3475 94) (width 0.3) (layer "F.Cu") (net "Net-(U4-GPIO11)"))
 (segment (start 138.1769 92.7813) (end 140 94) (width 0.3) (layer "F.Cu") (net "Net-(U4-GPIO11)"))
 (segment (start 126.4686 92.7813) (end 138.1769 92.7813) (width 0.3) (layer "F.Cu") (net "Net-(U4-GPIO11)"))
 (segment (start 143 102) (end 168 102) (width 0.3) (layer "F.Cu") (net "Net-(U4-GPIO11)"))
 (segment (start 168 102) (end 168.755 101) (width 0.3) (layer "F.Cu") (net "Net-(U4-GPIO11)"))
 (segment (start 168.755 101) (end 168.755 97.9125) (width 0.3048) (layer "F.Cu") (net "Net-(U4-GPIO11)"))
 (segment (start 140 94) (end 140 99) (width 0.3) (layer "F.Cu") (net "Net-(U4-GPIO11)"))
 (segment (start 140 99) (end 143 102) (width 0.3) (layer "F.Cu") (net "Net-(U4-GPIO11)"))
 (segment (start 123.884 90.1967) (end 126.4686 92.7813) (width 0.3) (layer "F.Cu") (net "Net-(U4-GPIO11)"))
 (segment (start 118.1022 90.1967) (end 123.884 90.1967) (width 0.3) (layer "F.Cu") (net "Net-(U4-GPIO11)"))
 (segment (start 119.22 96.54) (end 121.0925 96.54) (width 0.3) (layer "F.Cu") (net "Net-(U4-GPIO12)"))
 (segment (start 139 100.3499) (end 142 103) (width 0.3) (layer "F.Cu") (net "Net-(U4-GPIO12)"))
 (segment (start 171.272727 102) (end 171.295 101.977727) (width 0.3048) (layer "F.Cu") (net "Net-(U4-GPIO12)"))
 (segment (start 171.295 101.977727) (end 171.295 97.9125) (width 0.3048) (layer "F.Cu") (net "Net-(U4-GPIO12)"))
 (segment (start 121.0925 96.54) (end 124.9024 100.3499) (width 0.3) (layer "F.Cu") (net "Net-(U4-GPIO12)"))
 (segment (start 124.9024 100.3499) (end 139 100.3499) (width 0.3) (layer "F.Cu") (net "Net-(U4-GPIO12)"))
 (segment (start 170 103) (end 171.272727 102) (width 0.3) (layer "F.Cu") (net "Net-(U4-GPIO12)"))
 (segment (start 142 103) (end 170 103) (width 0.3) (layer "F.Cu") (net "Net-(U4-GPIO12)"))
 (segment (start 94.6534 65.8816) (end 93.17 67.365) (width 0.3) (layer "F.Cu") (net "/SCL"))
 (segment (start 119.3984 65.8816) (end 94.6534 65.8816) (width 0.3) (layer "F.Cu") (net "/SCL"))
 (segment (start 128.73 56.55) (end 119.3984 65.8816) (width 0.3) (layer "F.Cu") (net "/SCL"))
 (segment (start 168 57.0552) (end 168 70.7275) (width 0.3048) (layer "F.Cu") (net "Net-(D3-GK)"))
 (segment (start 168 70.7275) (end 163.675 75.0525) (width 0.3048) (layer "F.Cu") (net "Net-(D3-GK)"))
 (segment (start 166.47 56.73) (end 167.6748 56.73) (width 0.3048) (layer "F.Cu") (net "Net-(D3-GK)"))
 (segment (start 167.6748 56.73) (end 168 57.0552) (width 0.3048) (layer "F.Cu") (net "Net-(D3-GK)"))
 (segment (start 159 60.54) (end 160.4517 60.54) (width 0.3) (layer "F.Cu") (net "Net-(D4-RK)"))
 (segment (start 161.135 61.2233) (end 160.4517 60.54) (width 0.3) (layer "F.Cu") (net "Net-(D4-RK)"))
 (segment (start 161.135 75.0525) (end 161.135 61.2233) (width 0.3) (layer "F.Cu") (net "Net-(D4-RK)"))
 (segment (start 157.5483 74.0058) (end 157.5483 58) (width 0.3) (layer "F.Cu") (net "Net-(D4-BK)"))
 (segment (start 159 58) (end 157.5483 58) (width 0.3) (layer "F.Cu") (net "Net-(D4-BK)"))
 (segment (start 158.595 75.0525) (end 157.5483 74.0058) (width 0.3) (layer "F.Cu") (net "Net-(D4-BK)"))
 (segment (start 90.63 67.365) (end 102.4439 55.5511) (width 0.3) (layer "F.Cu") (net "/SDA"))
 (segment (start 84.1476 67.945894) (end 84.969106 68.7674) (width 0.3048) (layer "F.Cu") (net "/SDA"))
 (segment (start 102.4439 55.5511) (end 125.1911 55.5511) (width 0.3) (layer "F.Cu") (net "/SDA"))
 (segment (start 166.215 95.3725) (end 178 83.5875) (width 0.3048) (layer "F.Cu") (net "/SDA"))
 (segment (start 125.1911 55.5511) (end 126.19 56.55) (width 0.3) (layer "F.Cu") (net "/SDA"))
 (segment (start 178 63.771056) (end 168.261344 54.0324) (width 0.3048) (layer "F.Cu") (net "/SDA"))
 (segment (start 89.2276 68.7674) (end 90.63 67.365) (width 0.3048) (layer "F.Cu") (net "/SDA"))
 (segment (start 96.899306 54.0324) (end 84.1476 66.784106) (width 0.3048) (layer "F.Cu") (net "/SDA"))
 (segment (start 178 83.5875) (end 178 63.771056) (width 0.3048) (layer "F.Cu") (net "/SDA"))
 (segment (start 84.1476 66.784106) (end 84.1476 67.945894) (width 0.3048) (layer "F.Cu") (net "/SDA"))
 (segment (start 84.969106 68.7674) (end 89.2276 68.7674) (width 0.3048) (layer "F.Cu") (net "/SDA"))
 (segment (start 168.261344 54.0324) (end 96.899306 54.0324) (width 0.3048) (layer "F.Cu") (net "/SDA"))
 (segment (start 173.835 95.3725) (end 178 95.3725) (width 0.3048) (layer "F.Cu") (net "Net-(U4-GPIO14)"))
 (segment (start 181 99) (end 178 95.3725) (width 0.3) (layer "F.Cu") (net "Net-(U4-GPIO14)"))
 (segment (start 181 110.5) (end 181 99) (width 0.3) (layer "F.Cu") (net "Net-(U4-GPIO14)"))
 (segment (start 165.0183 56.1675) (end 165.5902 55.5956) (width 0.3) (layer "F.Cu") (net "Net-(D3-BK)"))
 (segment (start 175.9582 78.4448) (end 174.6746 79.7284) (width 0.3) (layer "F.Cu") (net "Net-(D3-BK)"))
 (segment (start 175.9582 63.7149) (end 175.9582 78.4448) (width 0.3) (layer "F.Cu") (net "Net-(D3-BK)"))
 (segment (start 166.47 58) (end 165.0183 58) (width 0.3) (layer "F.Cu") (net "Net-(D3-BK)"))
 (segment (start 167.8389 55.5956) (end 175.9582 63.7149) (width 0.3) (layer "F.Cu") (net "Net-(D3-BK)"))
 (segment (start 174.6746 79.7284) (end 165.8109 79.7284) (width 0.3) (layer "F.Cu") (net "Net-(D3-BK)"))
 (segment (start 165.0183 58) (end 165.0183 56.1675) (width 0.3) (layer "F.Cu") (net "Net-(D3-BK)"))
 (segment (start 165.8109 79.7284) (end 163.675 77.5925) (width 0.3) (layer "F.Cu") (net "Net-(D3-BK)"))
 (segment (start 165.5902 55.5956) (end 167.8389 55.5956) (width 0.3) (layer "F.Cu") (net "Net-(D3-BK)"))
 (segment (start 163.9762 80.4337) (end 161.135 77.5925) (width 0.3) (layer "F.Cu") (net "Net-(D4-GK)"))
 (segment (start 176.6739 63.4383) (end 176.6739 78.7816) (width 0.3) (layer "F.Cu") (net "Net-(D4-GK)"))
 (segment (start 176.6739 78.7816) (end 175.0218 80.4337) (width 0.3) (layer "F.Cu") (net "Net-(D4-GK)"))
 (segment (start 168.107 54.8714) (end 176.6739 63.4383) (width 0.3) (layer "F.Cu") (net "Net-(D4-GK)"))
 (segment (start 159 56.73) (end 160.4517 56.73) (width 0.3) (layer "F.Cu") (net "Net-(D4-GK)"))
 (segment (start 175.0218 80.4337) (end 163.9762 80.4337) (width 0.3) (layer "F.Cu") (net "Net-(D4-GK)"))
 (segment (start 162.3103 54.8714) (end 168.107 54.8714) (width 0.3) (layer "F.Cu") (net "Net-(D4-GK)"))
 (segment (start 160.4517 56.73) (end 162.3103 54.8714) (width 0.3) (layer "F.Cu") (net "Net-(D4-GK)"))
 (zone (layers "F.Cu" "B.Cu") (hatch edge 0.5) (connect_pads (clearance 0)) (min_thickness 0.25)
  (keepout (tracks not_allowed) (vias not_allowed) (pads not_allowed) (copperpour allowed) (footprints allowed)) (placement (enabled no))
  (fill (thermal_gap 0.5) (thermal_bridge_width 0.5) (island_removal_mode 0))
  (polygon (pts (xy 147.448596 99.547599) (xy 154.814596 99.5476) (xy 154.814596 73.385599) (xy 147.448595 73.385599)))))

